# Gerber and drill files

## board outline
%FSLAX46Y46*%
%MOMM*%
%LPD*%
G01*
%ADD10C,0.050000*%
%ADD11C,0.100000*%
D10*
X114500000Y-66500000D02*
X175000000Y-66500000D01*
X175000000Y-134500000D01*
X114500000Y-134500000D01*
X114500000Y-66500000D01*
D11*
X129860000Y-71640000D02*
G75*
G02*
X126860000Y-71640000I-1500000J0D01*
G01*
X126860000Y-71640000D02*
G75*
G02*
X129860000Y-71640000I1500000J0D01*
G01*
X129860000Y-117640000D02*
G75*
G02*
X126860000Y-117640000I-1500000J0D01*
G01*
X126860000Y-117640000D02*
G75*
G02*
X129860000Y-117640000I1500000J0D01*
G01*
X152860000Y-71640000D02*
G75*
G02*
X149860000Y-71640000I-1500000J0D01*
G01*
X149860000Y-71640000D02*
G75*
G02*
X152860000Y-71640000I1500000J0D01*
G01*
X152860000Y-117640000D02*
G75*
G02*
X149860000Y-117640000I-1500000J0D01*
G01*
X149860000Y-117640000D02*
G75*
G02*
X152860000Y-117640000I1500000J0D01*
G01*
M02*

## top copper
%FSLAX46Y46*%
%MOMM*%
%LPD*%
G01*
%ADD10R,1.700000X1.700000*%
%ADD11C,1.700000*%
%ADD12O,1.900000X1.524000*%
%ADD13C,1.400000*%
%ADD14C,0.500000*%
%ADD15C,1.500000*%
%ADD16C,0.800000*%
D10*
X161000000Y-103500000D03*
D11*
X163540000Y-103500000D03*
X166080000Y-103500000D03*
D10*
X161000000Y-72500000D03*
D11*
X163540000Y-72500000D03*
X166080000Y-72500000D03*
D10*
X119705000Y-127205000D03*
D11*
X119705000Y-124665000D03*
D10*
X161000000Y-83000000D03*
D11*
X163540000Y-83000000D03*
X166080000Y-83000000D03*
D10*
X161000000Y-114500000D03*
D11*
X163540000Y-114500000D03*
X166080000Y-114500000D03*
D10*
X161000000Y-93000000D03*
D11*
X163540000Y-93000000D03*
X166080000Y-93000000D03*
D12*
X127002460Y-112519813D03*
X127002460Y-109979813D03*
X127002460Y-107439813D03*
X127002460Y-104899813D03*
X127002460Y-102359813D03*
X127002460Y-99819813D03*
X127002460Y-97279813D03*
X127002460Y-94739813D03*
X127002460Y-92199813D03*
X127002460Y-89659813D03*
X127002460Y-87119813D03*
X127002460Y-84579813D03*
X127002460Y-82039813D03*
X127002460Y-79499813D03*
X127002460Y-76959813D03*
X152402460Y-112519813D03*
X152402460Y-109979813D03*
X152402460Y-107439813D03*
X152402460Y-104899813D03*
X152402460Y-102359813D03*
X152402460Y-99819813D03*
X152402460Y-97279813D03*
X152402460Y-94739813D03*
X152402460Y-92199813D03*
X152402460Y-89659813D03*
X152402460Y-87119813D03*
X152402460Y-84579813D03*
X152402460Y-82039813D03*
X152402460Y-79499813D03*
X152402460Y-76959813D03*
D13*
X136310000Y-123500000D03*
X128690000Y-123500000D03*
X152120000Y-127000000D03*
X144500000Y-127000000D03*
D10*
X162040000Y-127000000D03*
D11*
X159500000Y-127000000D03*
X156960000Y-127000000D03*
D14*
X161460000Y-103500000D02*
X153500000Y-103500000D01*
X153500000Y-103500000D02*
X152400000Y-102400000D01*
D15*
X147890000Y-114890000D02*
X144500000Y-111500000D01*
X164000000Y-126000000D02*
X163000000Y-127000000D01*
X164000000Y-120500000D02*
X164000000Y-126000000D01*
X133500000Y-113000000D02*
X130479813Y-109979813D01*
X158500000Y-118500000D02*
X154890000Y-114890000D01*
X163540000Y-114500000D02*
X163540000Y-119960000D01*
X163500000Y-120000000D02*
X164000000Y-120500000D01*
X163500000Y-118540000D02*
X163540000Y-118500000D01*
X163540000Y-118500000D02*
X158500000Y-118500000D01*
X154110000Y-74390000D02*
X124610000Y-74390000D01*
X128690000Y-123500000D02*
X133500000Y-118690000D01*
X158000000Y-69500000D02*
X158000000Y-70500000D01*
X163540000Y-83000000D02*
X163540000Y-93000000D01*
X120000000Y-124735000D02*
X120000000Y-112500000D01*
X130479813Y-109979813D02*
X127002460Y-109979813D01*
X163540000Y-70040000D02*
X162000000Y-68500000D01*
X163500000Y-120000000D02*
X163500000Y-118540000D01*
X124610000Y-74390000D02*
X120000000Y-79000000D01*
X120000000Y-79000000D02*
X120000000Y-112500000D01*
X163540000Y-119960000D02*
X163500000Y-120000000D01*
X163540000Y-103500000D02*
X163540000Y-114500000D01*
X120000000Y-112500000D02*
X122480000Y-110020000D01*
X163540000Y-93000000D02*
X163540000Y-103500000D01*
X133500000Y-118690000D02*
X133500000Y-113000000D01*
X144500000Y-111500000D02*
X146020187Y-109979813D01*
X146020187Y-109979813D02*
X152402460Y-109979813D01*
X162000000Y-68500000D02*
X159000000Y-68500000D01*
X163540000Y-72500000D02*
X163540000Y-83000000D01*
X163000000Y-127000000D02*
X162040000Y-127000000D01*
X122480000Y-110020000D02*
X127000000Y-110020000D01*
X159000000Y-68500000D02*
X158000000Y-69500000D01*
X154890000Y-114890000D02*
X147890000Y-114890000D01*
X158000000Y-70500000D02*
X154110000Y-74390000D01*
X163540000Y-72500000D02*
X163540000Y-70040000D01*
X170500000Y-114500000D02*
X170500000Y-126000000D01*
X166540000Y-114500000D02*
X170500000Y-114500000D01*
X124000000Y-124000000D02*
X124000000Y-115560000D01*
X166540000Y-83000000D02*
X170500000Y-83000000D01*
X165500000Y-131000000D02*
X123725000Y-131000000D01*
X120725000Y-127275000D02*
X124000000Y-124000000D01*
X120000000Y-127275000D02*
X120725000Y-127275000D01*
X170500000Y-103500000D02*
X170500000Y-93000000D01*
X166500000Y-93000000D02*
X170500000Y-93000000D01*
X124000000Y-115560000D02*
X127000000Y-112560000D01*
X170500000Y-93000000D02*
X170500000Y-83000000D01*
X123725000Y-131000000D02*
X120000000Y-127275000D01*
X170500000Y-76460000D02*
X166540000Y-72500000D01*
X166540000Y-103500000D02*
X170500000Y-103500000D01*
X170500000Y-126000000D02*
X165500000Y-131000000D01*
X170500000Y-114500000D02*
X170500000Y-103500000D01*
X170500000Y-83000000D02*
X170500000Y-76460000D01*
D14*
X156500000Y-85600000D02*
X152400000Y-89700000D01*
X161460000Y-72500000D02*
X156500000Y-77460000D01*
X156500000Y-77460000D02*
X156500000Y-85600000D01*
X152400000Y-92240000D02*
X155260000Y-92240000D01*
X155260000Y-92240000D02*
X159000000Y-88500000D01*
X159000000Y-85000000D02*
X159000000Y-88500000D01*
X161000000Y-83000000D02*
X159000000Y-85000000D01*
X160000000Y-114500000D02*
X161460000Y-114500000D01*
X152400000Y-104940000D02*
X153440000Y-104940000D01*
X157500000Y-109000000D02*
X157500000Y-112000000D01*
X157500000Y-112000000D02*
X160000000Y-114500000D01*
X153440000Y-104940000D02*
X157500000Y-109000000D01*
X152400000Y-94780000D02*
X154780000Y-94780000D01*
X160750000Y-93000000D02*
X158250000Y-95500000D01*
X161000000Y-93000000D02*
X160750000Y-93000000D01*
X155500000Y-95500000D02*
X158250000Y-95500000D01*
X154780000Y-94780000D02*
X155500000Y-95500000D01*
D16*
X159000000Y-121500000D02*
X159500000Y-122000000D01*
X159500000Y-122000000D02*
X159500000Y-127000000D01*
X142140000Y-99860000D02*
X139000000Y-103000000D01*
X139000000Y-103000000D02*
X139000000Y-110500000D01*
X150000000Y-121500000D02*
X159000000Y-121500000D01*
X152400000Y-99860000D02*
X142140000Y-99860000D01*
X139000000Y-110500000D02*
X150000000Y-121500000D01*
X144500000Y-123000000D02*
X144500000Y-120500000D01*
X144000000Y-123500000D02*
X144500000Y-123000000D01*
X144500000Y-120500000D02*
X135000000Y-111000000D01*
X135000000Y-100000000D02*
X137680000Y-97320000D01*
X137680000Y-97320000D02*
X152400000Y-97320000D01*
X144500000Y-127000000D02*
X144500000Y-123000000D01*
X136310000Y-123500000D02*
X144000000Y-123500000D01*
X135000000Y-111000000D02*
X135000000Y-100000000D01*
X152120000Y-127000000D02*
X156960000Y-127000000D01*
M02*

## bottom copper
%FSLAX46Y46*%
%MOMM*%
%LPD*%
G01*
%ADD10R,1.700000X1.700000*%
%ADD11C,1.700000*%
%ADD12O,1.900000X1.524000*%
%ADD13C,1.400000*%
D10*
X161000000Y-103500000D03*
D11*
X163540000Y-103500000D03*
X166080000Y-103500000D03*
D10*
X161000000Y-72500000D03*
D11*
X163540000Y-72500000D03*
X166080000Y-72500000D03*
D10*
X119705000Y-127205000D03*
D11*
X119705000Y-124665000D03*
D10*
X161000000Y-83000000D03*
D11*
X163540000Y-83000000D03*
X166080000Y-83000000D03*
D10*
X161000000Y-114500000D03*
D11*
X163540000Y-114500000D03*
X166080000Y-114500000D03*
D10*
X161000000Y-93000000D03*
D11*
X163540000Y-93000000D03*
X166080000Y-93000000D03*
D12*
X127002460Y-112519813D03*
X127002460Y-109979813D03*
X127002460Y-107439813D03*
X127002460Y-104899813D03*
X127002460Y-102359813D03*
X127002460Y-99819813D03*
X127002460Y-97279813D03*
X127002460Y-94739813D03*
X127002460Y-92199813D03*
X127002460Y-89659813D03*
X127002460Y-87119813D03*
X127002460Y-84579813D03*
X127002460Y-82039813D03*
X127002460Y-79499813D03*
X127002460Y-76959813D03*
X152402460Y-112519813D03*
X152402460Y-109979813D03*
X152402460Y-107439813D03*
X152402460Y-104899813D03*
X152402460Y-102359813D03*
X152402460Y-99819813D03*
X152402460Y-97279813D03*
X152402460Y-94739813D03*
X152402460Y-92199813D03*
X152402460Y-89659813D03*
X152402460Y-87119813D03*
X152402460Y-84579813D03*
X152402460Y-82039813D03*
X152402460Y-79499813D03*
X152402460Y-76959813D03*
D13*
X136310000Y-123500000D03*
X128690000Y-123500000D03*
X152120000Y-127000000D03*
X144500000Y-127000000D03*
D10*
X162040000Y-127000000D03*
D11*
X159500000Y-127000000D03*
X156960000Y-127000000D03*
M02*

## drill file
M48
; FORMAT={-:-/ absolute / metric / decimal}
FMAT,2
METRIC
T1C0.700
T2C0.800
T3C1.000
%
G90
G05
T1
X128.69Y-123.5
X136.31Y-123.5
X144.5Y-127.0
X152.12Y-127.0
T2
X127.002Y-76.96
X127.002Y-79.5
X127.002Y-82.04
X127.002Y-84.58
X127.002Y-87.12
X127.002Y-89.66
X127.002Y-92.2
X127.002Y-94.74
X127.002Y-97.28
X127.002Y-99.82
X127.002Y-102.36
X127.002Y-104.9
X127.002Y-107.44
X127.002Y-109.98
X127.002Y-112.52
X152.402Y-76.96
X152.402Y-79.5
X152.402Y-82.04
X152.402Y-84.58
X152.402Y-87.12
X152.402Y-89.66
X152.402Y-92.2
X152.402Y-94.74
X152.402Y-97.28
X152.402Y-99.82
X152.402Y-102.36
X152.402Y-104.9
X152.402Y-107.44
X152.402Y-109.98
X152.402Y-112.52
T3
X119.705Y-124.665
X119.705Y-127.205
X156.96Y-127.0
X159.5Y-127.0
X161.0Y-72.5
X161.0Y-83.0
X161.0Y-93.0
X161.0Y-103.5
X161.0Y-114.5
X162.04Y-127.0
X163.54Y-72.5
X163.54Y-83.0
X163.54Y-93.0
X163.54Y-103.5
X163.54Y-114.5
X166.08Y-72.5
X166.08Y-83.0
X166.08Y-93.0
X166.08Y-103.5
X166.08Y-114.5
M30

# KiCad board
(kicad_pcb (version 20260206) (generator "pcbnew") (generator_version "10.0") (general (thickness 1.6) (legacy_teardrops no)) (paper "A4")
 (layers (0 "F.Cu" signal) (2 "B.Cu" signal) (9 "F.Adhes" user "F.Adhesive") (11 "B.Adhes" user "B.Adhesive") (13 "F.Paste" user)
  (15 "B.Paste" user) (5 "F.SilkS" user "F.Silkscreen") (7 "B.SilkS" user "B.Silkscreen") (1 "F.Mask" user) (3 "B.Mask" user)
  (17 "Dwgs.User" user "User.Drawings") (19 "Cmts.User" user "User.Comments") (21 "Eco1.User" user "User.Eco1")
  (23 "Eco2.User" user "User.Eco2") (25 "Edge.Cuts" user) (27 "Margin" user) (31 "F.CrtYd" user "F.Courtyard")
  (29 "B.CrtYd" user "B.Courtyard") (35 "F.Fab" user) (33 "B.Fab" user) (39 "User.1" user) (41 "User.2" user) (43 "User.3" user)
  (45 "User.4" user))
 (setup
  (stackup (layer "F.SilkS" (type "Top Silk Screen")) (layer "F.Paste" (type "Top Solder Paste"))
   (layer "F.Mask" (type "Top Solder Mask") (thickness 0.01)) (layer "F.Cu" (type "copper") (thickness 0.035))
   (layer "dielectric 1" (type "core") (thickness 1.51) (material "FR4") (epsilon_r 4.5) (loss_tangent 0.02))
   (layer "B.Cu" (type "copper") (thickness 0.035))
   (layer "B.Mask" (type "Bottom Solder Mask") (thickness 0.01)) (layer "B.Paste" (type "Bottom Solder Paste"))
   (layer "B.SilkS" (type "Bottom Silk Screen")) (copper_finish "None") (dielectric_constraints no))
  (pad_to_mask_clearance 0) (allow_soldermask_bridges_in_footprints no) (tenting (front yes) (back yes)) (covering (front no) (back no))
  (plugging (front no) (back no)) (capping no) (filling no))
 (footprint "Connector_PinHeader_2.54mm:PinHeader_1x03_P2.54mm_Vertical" (layer "F.Cu") (at 161 103.5 90)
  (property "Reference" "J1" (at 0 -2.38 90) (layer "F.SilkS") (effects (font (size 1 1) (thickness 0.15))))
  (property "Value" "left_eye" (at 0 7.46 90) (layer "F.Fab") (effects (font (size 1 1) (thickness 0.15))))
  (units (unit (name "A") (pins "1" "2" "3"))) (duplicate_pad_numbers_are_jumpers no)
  (pad "1" thru_hole rect (at 0 0 90) (size 1.7 1.7) (drill 1) (layers "*.Cu" "*.Mask") (remove_unused_layers no) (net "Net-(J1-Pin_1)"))
  (pad "2" thru_hole circle (at 0 2.54 90) (size 1.7 1.7) (drill 1) (layers "*.Cu" "*.Mask") (remove_unused_layers no) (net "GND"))
  (pad "3" thru_hole circle (at 0 5.08 90) (size 1.7 1.7) (drill 1) (layers "*.Cu" "*.Mask") (remove_unused_layers no) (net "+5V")))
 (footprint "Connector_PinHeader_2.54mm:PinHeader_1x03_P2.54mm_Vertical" (layer "F.Cu") (at 161 72.5 90)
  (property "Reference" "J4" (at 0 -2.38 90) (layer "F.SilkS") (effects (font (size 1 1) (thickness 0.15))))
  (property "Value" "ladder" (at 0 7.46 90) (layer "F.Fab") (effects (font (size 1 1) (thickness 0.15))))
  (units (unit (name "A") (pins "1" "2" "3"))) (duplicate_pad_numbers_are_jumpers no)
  (pad "1" thru_hole rect (at 0 0 90) (size 1.7 1.7) (drill 1) (layers "*.Cu" "*.Mask") (remove_unused_layers no) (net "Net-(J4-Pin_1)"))
  (pad "2" thru_hole circle (at 0 2.54 90) (size 1.7 1.7) (drill 1) (layers "*.Cu" "*.Mask") (remove_unused_layers no) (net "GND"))
  (pad "3" thru_hole circle (at 0 5.08 90) (size 1.7 1.7) (drill 1) (layers "*.Cu" "*.Mask") (remove_unused_layers no) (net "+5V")))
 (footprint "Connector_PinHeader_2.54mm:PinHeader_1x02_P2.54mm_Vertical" (layer "F.Cu") (at 119.705 127.205 180)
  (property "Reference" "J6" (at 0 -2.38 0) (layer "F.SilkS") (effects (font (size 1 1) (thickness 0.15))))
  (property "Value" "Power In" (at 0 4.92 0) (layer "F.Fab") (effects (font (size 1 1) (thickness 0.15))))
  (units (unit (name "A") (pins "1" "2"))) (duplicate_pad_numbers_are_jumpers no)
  (pad "1" thru_hole rect (at 0 0 180) (size 1.7 1.7) (drill 1) (layers "*.Cu" "*.Mask") (remove_unused_layers no) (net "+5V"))
  (pad "2" thru_hole circle (at 0 2.54 180) (size 1.7 1.7) (drill 1) (layers "*.Cu" "*.Mask") (remove_unused_layers no) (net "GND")))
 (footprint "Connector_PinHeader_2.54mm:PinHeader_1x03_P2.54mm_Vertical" (layer "F.Cu") (at 161 83 90)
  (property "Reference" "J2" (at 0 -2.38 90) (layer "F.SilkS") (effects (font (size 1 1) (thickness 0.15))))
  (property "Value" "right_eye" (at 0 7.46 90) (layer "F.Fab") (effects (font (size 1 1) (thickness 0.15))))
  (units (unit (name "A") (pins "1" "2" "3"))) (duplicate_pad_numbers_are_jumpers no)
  (pad "1" thru_hole rect (at 0 0 90) (size 1.7 1.7) (drill 1) (layers "*.Cu" "*.Mask") (remove_unused_layers no) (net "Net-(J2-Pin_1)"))
  (pad "2" thru_hole circle (at 0 2.54 90) (size 1.7 1.7) (drill 1) (layers "*.Cu" "*.Mask") (remove_unused_layers no) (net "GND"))
  (pad "3" thru_hole circle (at 0 5.08 90) (size 1.7 1.7) (drill 1) (layers "*.Cu" "*.Mask") (remove_unused_layers no) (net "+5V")))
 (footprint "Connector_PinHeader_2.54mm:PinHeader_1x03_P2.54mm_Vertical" (layer "F.Cu") (at 161 114.5 90)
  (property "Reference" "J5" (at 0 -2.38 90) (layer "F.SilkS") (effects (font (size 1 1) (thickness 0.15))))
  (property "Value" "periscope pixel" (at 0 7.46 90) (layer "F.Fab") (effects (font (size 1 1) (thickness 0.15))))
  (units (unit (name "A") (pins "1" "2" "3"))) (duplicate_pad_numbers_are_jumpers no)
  (pad "1" thru_hole rect (at 0 0 90) (size 1.7 1.7) (drill 1) (layers "*.Cu" "*.Mask") (remove_unused_layers no) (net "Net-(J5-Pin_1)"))
  (pad "2" thru_hole circle (at 0 2.54 90) (size 1.7 1.7) (drill 1) (layers "*.Cu" "*.Mask") (remove_unused_layers no) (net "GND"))
  (pad "3" thru_hole circle (at 0 5.08 90) (size 1.7 1.7) (drill 1) (layers "*.Cu" "*.Mask") (remove_unused_layers no) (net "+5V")))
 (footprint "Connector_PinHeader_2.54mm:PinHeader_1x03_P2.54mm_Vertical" (layer "F.Cu") (at 161 93 90)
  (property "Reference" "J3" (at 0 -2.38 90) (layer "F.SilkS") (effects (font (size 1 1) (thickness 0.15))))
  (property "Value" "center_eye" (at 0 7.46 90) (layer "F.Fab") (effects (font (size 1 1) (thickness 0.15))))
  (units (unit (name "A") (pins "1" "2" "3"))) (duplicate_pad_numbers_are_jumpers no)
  (pad "1" thru_hole rect (at 0 0 90) (size 1.7 1.7) (drill 1) (layers "*.Cu" "*.Mask") (remove_unused_layers no) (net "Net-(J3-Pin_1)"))
  (pad "2" thru_hole circle (at 0 2.54 90) (size 1.7 1.7) (drill 1) (layers "*.Cu" "*.Mask") (remove_unused_layers no) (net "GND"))
  (pad "3" thru_hole circle (at 0 5.08 90) (size 1.7 1.7) (drill 1) (layers "*.Cu" "*.Mask") (remove_unused_layers no) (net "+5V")))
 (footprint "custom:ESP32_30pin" (layer "F.Cu") (at 138.93 95.5)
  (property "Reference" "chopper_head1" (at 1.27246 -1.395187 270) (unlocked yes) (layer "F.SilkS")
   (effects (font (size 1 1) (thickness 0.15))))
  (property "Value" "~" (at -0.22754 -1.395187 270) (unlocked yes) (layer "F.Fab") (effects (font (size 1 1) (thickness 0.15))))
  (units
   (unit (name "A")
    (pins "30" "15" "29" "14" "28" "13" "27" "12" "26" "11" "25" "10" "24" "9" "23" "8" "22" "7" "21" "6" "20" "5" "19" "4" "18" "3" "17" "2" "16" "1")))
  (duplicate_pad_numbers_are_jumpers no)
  (fp_circle (center -10.57 -23.86) (end -10.57 -22.36) (stroke (width 0.1) (type default)) (fill no) (layer "Edge.Cuts"))
  (fp_circle (center -10.57 22.14) (end -10.57 23.64) (stroke (width 0.1) (type default)) (fill no) (layer "Edge.Cuts"))
  (fp_circle (center 12.43 -23.86) (end 12.43 -22.36) (stroke (width 0.1) (type default)) (fill no) (layer "Edge.Cuts"))
  (fp_circle (center 12.43 22.14) (end 12.43 23.64) (stroke (width 0.1) (type default)) (fill no) (layer "Edge.Cuts"))
  (pad "1" thru_hole oval (at -11.92754 17.019813 270) (size 1.524 1.9) (drill 0.8) (layers "*.Cu" "*.Mask") (remove_unused_layers no)
   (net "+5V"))
  (pad "2" thru_hole oval (at -11.92754 14.479813 270) (size 1.524 1.9) (drill 0.8) (layers "*.Cu" "*.Mask") (remove_unused_layers no)
   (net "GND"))
  (pad "3" thru_hole oval (at -11.92754 11.939813 270) (size 1.524 1.9) (drill 0.8) (layers "*.Cu" "*.Mask") (remove_unused_layers no)
   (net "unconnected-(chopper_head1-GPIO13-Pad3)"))
  (pad "4" thru_hole oval (at -11.92754 9.399813 270) (size 1.524 1.9) (drill 0.8) (layers "*.Cu" "*.Mask") (remove_unused_layers no)
   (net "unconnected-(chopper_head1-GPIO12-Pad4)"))
  (pad "5" thru_hole oval (at -11.92754 6.859813 270) (size 1.524 1.9) (drill 0.8) (layers "*.Cu" "*.Mask") (remove_unused_layers no)
   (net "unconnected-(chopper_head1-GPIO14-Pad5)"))
  (pad "6" thru_hole oval (at -11.92754 4.319813 270) (size 1.524 1.9) (drill 0.8) (layers "*.Cu" "*.Mask") (remove_unused_layers no)
   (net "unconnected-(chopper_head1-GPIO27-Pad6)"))
  (pad "7" thru_hole oval (at -11.92754 1.779813 270) (size 1.524 1.9) (drill 0.8) (layers "*.Cu" "*.Mask") (remove_unused_layers no)
   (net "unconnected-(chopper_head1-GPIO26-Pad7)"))
  (pad "8" thru_hole oval (at -11.92754 -0.760187 270) (size 1.524 1.9) (drill 0.8) (layers "*.Cu" "*.Mask") (remove_unused_layers no)
   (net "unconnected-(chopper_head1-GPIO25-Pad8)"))
  (pad "9" thru_hole oval (at -11.92754 -3.300187 270) (size 1.524 1.9) (drill 0.8) (layers "*.Cu" "*.Mask") (remove_unused_layers no)
   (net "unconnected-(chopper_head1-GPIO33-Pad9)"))
  (pad "10" thru_hole oval (at -11.92754 -5.840187 270) (size 1.524 1.9) (drill 0.8) (layers "*.Cu" "*.Mask") (remove_unused_layers no)
   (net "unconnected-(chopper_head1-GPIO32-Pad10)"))
  (pad "11" thru_hole oval (at -11.92754 -8.380187 270) (size 1.524 1.9) (drill 0.8) (layers "*.Cu" "*.Mask") (remove_unused_layers no)
   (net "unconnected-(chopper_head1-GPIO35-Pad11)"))
  (pad "12" thru_hole oval (at -11.92754 -10.920187 270) (size 1.524 1.9) (drill 0.8) (layers "*.Cu" "*.Mask") (remove_unused_layers no)
   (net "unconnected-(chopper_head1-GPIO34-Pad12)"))
  (pad "13" thru_hole oval (at -11.92754 -13.460187 270) (size 1.524 1.9) (drill 0.8) (layers "*.Cu" "*.Mask") (remove_unused_layers no)
   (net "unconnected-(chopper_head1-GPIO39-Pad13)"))
  (pad "14" thru_hole oval (at -11.92754 -16.000187 270) (size 1.524 1.9) (drill 0.8) (layers "*.Cu" "*.Mask") (remove_unused_layers no)
   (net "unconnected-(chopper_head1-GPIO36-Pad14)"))
  (pad "15" thru_hole oval (at -11.92754 -18.540187 270) (size 1.524 1.9) (drill 0.8) (layers "*.Cu" "*.Mask") (remove_unused_layers no)
   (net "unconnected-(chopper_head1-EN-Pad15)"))
  (pad "16" thru_hole oval (at 13.47246 17.019813 270) (size 1.524 1.9) (drill 0.8) (layers "*.Cu" "*.Mask") (remove_unused_layers no)
   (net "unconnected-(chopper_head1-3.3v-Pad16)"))
  (pad "17" thru_hole oval (at 13.47246 14.479813 270) (size 1.524 1.9) (drill 0.8) (layers "*.Cu" "*.Mask") (remove_unused_layers no)
   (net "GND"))
  (pad "18" thru_hole oval (at 13.47246 11.939813 270) (size 1.524 1.9) (drill 0.8) (layers "*.Cu" "*.Mask") (remove_unused_layers no)
   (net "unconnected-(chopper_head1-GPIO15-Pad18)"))
  (pad "19" thru_hole oval (at 13.47246 9.399813 270) (size 1.524 1.9) (drill 0.8) (layers "*.Cu" "*.Mask") (remove_unused_layers no)
   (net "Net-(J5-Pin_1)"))
  (pad "20" thru_hole oval (at 13.47246 6.859813 270) (size 1.524 1.9) (drill 0.8) (layers "*.Cu" "*.Mask" "Dwgs.User")
   (remove_unused_layers no) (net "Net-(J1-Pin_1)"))
  (pad "21" thru_hole oval (at 13.47246 4.319813 270) (size 1.524 1.9) (drill 0.8) (layers "*.Cu" "*.Mask") (remove_unused_layers no)
   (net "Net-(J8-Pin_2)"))
  (pad "22" thru_hole oval (at 13.47246 1.779813 270) (size 1.524 1.9) (drill 0.8) (layers "*.Cu" "*.Mask") (remove_unused_layers no)
   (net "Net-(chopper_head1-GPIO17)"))
  (pad "23" thru_hole oval (at 13.47246 -0.760187 270) (size 1.524 1.9) (drill 0.8) (layers "*.Cu" "*.Mask") (remove_unused_layers no)
   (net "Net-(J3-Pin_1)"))
  (pad "24" thru_hole oval (at 13.47246 -3.300187 270) (size 1.524 1.9) (drill 0.8) (layers "*.Cu" "*.Mask") (remove_unused_layers no)
   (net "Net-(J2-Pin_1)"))
  (pad "25" thru_hole oval (at 13.47246 -5.840187 270) (size 1.524 1.9) (drill 0.8) (layers "*.Cu" "*.Mask") (remove_unused_layers no)
   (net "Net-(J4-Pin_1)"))
  (pad "26" thru_hole oval (at 13.47246 -8.380187 270) (size 1.524 1.9) (drill 0.8) (layers "*.Cu" "*.Mask") (remove_unused_layers no)
   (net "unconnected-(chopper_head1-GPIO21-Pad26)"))
  (pad "27" thru_hole oval (at 13.47246 -10.920187 270) (size 1.524 1.9) (drill 0.8) (layers "*.Cu" "*.Mask") (remove_unused_layers no)
   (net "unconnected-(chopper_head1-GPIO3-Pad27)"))
  (pad "28" thru_hole oval (at 13.47246 -13.460187 270) (size 1.524 1.9) (drill 0.8) (layers "*.Cu" "*.Mask") (remove_unused_layers no)
   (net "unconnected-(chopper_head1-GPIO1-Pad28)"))
  (pad "29" thru_hole oval (at 13.47246 -16.000187 270) (size 1.524 1.9) (drill 0.8) (layers "*.Cu" "*.Mask") (remove_unused_layers no)
   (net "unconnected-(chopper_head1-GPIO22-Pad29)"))
  (pad "30" thru_hole oval (at 13.47246 -18.540187 270) (size 1.524 1.9) (drill 0.8) (layers "*.Cu" "*.Mask") (remove_unused_layers no)
   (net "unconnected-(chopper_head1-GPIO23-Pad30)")))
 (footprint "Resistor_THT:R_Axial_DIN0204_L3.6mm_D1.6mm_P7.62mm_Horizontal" (layer "F.Cu") (at 136.31 123.5 180)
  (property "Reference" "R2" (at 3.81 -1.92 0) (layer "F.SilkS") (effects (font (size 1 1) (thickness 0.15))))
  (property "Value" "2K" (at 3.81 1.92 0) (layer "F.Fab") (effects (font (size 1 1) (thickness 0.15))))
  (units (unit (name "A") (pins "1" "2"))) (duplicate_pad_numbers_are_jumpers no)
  (pad "1" thru_hole circle (at 0 0 180) (size 1.4 1.4) (drill 0.7) (layers "*.Cu" "*.Mask") (remove_unused_layers no)
   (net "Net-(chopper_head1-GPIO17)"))
  (pad "2" thru_hole circle (at 7.62 0 180) (size 1.4 1.4) (drill 0.7) (layers "*.Cu" "*.Mask") (remove_unused_layers no) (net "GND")))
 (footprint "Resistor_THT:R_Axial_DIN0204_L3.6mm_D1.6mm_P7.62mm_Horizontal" (layer "F.Cu") (at 152.12 127 180)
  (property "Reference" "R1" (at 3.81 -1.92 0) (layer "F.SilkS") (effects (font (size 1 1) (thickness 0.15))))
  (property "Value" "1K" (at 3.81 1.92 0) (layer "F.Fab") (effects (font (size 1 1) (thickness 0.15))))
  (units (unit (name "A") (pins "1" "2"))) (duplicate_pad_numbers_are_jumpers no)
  (pad "1" thru_hole circle (at 0 0 180) (size 1.4 1.4) (drill 0.7) (layers "*.Cu" "*.Mask") (remove_unused_layers no)
   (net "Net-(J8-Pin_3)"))
  (pad "2" thru_hole circle (at 7.62 0 180) (size 1.4 1.4) (drill 0.7) (layers "*.Cu" "*.Mask") (remove_unused_layers no)
   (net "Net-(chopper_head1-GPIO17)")))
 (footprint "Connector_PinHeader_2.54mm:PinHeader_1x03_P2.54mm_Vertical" (layer "F.Cu") (at 162.04 127 -90)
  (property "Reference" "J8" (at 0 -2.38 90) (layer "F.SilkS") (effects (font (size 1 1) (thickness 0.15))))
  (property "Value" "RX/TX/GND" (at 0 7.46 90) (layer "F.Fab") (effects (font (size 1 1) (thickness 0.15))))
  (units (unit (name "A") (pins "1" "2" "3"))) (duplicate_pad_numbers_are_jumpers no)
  (pad "1" thru_hole rect (at 0 0 270) (size 1.7 1.7) (drill 1) (layers "*.Cu" "*.Mask") (remove_unused_layers no) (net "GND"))
  (pad "2" thru_hole circle (at 0 2.54 270) (size 1.7 1.7) (drill 1) (layers "*.Cu" "*.Mask") (remove_unused_layers no)
   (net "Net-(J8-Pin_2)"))
  (pad "3" thru_hole circle (at 0 5.08 270) (size 1.7 1.7) (drill 1) (layers "*.Cu" "*.Mask") (remove_unused_layers no)
   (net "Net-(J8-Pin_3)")))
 (gr_rect (start 114.5 66.5) (end 175 134.5) (stroke (width 0.05) (type default)) (fill no) (layer "Edge.Cuts"))
 (segment (start 161.46 103.5) (end 153.5 103.5) (width 0.5) (layer "F.Cu") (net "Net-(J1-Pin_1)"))
 (segment (start 153.5 103.5) (end 152.4 102.4) (width 0.5) (layer "F.Cu") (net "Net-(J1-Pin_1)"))
 (segment (start 147.89 114.89) (end 144.5 111.5) (width 1.5) (layer "F.Cu") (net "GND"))
 (segment (start 164 126) (end 163 127) (width 1.5) (layer "F.Cu") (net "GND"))
 (segment (start 164 120.5) (end 164 126) (width 1.5) (layer "F.Cu") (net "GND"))
 (segment (start 133.5 113) (end 130.479813 109.979813) (width 1.5) (layer "F.Cu") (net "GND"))
 (segment (start 158.5 118.5) (end 154.89 114.89) (width 1.5) (layer "F.Cu") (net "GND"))
 (segment (start 163.54 114.5) (end 163.54 119.96) (width 1.5) (layer "F.Cu") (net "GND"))
 (segment (start 163.5 120) (end 164 120.5) (width 1.5) (layer "F.Cu") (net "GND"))
 (segment (start 163.5 118.54) (end 163.54 118.5) (width 1.5) (layer "F.Cu") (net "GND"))
 (segment (start 163.54 118.5) (end 158.5 118.5) (width 1.5) (layer "F.Cu") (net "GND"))
 (segment (start 154.11 74.39) (end 124.61 74.39) (width 1.5) (layer "F.Cu") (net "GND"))
 (segment (start 128.69 123.5) (end 133.5 118.69) (width 1.5) (layer "F.Cu") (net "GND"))
 (segment (start 158 69.5) (end 158 70.5) (width 1.5) (layer "F.Cu") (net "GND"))
 (segment (start 163.54 83) (end 163.54 93) (width 1.5) (layer "F.Cu") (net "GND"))
 (segment (start 120 124.735) (end 120 112.5) (width 1.5) (layer "F.Cu") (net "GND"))
 (segment (start 130.479813 109.979813) (end 127.00246 109.979813) (width 1.5) (layer "F.Cu") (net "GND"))
 (segment (start 163.54 70.04) (end 162 68.5) (width 1.5) (layer "F.Cu") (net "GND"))
 (segment (start 163.5 120) (end 163.5 118.54) (width 1.5) (layer "F.Cu") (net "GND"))
 (segment (start 124.61 74.39) (end 120 79) (width 1.5) (layer "F.Cu") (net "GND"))
 (segment (start 120 79) (end 120 112.5) (width 1.5) (layer "F.Cu") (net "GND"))
 (segment (start 163.54 119.96) (end 163.5 120) (width 1.5) (layer "F.Cu") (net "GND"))
 (segment (start 163.54 103.5) (end 163.54 114.5) (width 1.5) (layer "F.Cu") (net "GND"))
 (segment (start 120 112.5) (end 122.48 110.02) (width 1.5) (layer "F.Cu") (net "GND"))
 (segment (start 163.54 93) (end 163.54 103.5) (width 1.5) (layer "F.Cu") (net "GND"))
 (segment (start 133.5 118.69) (end 133.5 113) (width 1.5) (layer "F.Cu") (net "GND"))
 (segment (start 144.5 111.5) (end 146.020187 109.979813) (width 1.5) (layer "F.Cu") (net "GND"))
 (segment (start 146.020187 109.979813) (end 152.40246 109.979813) (width 1.5) (layer "F.Cu") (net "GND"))
 (segment (start 162 68.5) (end 159 68.5) (width 1.5) (layer "F.Cu") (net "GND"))
 (segment (start 163.54 72.5) (end 163.54 83) (width 1.5) (layer "F.Cu") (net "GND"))
 (segment (start 163 127) (end 162.04 127) (width 1.5) (layer "F.Cu") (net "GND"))
 (segment (start 122.48 110.02) (end 127 110.02) (width 1.5) (layer "F.Cu") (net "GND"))
 (segment (start 159 68.5) (end 158 69.5) (width 1.5) (layer "F.Cu") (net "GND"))
 (segment (start 154.89 114.89) (end 147.89 114.89) (width 1.5) (layer "F.Cu") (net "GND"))
 (segment (start 158 70.5) (end 154.11 74.39) (width 1.5) (layer "F.Cu") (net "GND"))
 (segment (start 163.54 72.5) (end 163.54 70.04) (width 1.5) (layer "F.Cu") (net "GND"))
 (segment (start 170.5 114.5) (end 170.5 126) (width 1.5) (layer "F.Cu") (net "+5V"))
 (segment (start 166.54 114.5) (end 170.5 114.5) (width 1.5) (layer "F.Cu") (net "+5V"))
 (segment (start 124 124) (end 124 115.56) (width 1.5) (layer "F.Cu") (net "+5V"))
 (segment (start 166.54 83) (end 170.5 83) (width 1.5) (layer "F.Cu") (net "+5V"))
 (segment (start 165.5 131) (end 123.725 131) (width 1.5) (layer "F.Cu") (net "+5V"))
 (segment (start 120.725 127.275) (end 124 124) (width 1.5) (layer "F.Cu") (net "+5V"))
 (segment (start 120 127.275) (end 120.725 127.275) (width 1.5) (layer "F.Cu") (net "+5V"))
 (segment (start 170.5 103.5) (end 170.5 93) (width 1.5) (layer "F.Cu") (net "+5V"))
 (segment (start 166.5 93) (end 170.5 93) (width 1.5) (layer "F.Cu") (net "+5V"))
 (segment (start 124 115.56) (end 127 112.56) (width 1.5) (layer "F.Cu") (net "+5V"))
 (segment (start 170.5 93) (end 170.5 83) (width 1.5) (layer "F.Cu") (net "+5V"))
 (segment (start 123.725 131) (end 120 127.275) (width 1.5) (layer "F.Cu") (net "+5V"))
 (segment (start 170.5 76.46) (end 166.54 72.5) (width 1.5) (layer "F.Cu") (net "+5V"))
 (segment (start 166.54 103.5) (end 170.5 103.5) (width 1.5) (layer "F.Cu") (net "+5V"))
 (segment (start 170.5 126) (end 165.5 131) (width 1.5) (layer "F.Cu") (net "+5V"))
 (segment (start 170.5 114.5) (end 170.5 103.5) (width 1.5) (layer "F.Cu") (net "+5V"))
 (segment (start 170.5 83) (end 170.5 76.46) (width 1.5) (layer "F.Cu") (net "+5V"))
 (segment (start 156.5 85.6) (end 152.4 89.7) (width 0.5) (layer "F.Cu") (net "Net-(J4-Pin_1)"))
 (segment (start 161.46 72.5) (end 156.5 77.46) (width 0.5) (layer "F.Cu") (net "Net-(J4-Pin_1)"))
 (segment (start 156.5 77.46) (end 156.5 85.6) (width 0.5) (layer "F.Cu") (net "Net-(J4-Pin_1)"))
 (segment (start 152.4 92.24) (end 155.26 92.24) (width 0.5) (layer "F.Cu") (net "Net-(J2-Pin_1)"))
 (segment (start 155.26 92.24) (end 159 88.5) (width 0.5) (layer "F.Cu") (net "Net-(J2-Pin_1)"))
 (segment (start 159 85) (end 159 88.5) (width 0.5) (layer "F.Cu") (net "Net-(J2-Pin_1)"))
 (segment (start 161 83) (end 159 85) (width 0.5) (layer "F.Cu") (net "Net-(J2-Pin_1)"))
 (segment (start 160 114.5) (end 161.46 114.5) (width 0.5) (layer "F.Cu") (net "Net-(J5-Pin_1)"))
 (segment (start 152.4 104.94) (end 153.44 104.94) (width 0.5) (layer "F.Cu") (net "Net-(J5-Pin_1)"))
 (segment (start 157.5 109) (end 157.5 112) (width 0.5) (layer "F.Cu") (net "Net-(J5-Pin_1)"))
 (segment (start 157.5 112) (end 160 114.5) (width 0.5) (layer "F.Cu") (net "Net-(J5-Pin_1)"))
 (segment (start 153.44 104.94) (end 157.5 109) (width 0.5) (layer "F.Cu") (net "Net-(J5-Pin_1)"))
 (segment (start 152.4 94.78) (end 154.78 94.78) (width 0.5) (layer "F.Cu") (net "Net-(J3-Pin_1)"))
 (segment (start 160.75 93) (end 158.25 95.5) (width 0.5) (layer "F.Cu") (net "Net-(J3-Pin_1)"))
 (segment (start 161 93) (end 160.75 93) (width 0.5) (layer "F.Cu") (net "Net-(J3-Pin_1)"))
 (segment (start 155.5 95.5) (end 158.25 95.5) (width 0.5) (layer "F.Cu") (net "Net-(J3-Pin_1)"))
 (segment (start 154.78 94.78) (end 155.5 95.5) (width 0.5) (layer "F.Cu") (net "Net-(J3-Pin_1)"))
 (segment (start 159 121.5) (end 159.5 122) (width 0.8) (layer "F.Cu") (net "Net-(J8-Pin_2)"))
 (segment (start 159.5 122) (end 159.5 127) (width 0.8) (layer "F.Cu") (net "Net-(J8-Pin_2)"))
 (segment (start 142.14 99.86) (end 139 103) (width 0.8) (layer "F.Cu") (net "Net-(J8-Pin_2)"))
 (segment (start 139 103) (end 139 110.5) (width 0.8) (layer "F.Cu") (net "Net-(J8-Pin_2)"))
 (segment (start 150 121.5) (end 159 121.5) (width 0.8) (layer "F.Cu") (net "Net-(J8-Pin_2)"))
 (segment (start 152.4 99.86) (end 142.14 99.86) (width 0.8) (layer "F.Cu") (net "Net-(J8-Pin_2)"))
 (segment (start 139 110.5) (end 150 121.5) (width 0.8) (layer "F.Cu") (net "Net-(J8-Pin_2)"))
 (segment (start 144.5 123) (end 144.5 120.5) (width 0.8) (layer "F.Cu") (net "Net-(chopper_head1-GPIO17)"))
 (segment (start 144 123.5) (end 144.5 123) (width 0.8) (layer "F.Cu") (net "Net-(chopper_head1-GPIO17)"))
 (segment (start 144.5 120.5) (end 135 111) (width 0.8) (layer "F.Cu") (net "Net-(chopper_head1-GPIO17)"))
 (segment (start 135 100) (end 137.68 97.32) (width 0.8) (layer "F.Cu") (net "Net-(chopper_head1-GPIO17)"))
 (segment (start 137.68 97.32) (end 152.4 97.32) (width 0.8) (layer "F.Cu") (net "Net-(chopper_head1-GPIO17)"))
 (segment (start 144.5 127) (end 144.5 123) (width 0.8) (layer "F.Cu") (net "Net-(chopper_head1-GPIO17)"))
 (segment (start 136.31 123.5) (end 144 123.5) (width 0.8) (layer "F.Cu") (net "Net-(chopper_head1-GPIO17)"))
 (segment (start 135 111) (end 135 100) (width 0.8) (layer "F.Cu") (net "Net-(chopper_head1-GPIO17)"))
 (segment (start 152.12 127) (end 156.96 127) (width 0.8) (layer "F.Cu") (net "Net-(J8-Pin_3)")))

